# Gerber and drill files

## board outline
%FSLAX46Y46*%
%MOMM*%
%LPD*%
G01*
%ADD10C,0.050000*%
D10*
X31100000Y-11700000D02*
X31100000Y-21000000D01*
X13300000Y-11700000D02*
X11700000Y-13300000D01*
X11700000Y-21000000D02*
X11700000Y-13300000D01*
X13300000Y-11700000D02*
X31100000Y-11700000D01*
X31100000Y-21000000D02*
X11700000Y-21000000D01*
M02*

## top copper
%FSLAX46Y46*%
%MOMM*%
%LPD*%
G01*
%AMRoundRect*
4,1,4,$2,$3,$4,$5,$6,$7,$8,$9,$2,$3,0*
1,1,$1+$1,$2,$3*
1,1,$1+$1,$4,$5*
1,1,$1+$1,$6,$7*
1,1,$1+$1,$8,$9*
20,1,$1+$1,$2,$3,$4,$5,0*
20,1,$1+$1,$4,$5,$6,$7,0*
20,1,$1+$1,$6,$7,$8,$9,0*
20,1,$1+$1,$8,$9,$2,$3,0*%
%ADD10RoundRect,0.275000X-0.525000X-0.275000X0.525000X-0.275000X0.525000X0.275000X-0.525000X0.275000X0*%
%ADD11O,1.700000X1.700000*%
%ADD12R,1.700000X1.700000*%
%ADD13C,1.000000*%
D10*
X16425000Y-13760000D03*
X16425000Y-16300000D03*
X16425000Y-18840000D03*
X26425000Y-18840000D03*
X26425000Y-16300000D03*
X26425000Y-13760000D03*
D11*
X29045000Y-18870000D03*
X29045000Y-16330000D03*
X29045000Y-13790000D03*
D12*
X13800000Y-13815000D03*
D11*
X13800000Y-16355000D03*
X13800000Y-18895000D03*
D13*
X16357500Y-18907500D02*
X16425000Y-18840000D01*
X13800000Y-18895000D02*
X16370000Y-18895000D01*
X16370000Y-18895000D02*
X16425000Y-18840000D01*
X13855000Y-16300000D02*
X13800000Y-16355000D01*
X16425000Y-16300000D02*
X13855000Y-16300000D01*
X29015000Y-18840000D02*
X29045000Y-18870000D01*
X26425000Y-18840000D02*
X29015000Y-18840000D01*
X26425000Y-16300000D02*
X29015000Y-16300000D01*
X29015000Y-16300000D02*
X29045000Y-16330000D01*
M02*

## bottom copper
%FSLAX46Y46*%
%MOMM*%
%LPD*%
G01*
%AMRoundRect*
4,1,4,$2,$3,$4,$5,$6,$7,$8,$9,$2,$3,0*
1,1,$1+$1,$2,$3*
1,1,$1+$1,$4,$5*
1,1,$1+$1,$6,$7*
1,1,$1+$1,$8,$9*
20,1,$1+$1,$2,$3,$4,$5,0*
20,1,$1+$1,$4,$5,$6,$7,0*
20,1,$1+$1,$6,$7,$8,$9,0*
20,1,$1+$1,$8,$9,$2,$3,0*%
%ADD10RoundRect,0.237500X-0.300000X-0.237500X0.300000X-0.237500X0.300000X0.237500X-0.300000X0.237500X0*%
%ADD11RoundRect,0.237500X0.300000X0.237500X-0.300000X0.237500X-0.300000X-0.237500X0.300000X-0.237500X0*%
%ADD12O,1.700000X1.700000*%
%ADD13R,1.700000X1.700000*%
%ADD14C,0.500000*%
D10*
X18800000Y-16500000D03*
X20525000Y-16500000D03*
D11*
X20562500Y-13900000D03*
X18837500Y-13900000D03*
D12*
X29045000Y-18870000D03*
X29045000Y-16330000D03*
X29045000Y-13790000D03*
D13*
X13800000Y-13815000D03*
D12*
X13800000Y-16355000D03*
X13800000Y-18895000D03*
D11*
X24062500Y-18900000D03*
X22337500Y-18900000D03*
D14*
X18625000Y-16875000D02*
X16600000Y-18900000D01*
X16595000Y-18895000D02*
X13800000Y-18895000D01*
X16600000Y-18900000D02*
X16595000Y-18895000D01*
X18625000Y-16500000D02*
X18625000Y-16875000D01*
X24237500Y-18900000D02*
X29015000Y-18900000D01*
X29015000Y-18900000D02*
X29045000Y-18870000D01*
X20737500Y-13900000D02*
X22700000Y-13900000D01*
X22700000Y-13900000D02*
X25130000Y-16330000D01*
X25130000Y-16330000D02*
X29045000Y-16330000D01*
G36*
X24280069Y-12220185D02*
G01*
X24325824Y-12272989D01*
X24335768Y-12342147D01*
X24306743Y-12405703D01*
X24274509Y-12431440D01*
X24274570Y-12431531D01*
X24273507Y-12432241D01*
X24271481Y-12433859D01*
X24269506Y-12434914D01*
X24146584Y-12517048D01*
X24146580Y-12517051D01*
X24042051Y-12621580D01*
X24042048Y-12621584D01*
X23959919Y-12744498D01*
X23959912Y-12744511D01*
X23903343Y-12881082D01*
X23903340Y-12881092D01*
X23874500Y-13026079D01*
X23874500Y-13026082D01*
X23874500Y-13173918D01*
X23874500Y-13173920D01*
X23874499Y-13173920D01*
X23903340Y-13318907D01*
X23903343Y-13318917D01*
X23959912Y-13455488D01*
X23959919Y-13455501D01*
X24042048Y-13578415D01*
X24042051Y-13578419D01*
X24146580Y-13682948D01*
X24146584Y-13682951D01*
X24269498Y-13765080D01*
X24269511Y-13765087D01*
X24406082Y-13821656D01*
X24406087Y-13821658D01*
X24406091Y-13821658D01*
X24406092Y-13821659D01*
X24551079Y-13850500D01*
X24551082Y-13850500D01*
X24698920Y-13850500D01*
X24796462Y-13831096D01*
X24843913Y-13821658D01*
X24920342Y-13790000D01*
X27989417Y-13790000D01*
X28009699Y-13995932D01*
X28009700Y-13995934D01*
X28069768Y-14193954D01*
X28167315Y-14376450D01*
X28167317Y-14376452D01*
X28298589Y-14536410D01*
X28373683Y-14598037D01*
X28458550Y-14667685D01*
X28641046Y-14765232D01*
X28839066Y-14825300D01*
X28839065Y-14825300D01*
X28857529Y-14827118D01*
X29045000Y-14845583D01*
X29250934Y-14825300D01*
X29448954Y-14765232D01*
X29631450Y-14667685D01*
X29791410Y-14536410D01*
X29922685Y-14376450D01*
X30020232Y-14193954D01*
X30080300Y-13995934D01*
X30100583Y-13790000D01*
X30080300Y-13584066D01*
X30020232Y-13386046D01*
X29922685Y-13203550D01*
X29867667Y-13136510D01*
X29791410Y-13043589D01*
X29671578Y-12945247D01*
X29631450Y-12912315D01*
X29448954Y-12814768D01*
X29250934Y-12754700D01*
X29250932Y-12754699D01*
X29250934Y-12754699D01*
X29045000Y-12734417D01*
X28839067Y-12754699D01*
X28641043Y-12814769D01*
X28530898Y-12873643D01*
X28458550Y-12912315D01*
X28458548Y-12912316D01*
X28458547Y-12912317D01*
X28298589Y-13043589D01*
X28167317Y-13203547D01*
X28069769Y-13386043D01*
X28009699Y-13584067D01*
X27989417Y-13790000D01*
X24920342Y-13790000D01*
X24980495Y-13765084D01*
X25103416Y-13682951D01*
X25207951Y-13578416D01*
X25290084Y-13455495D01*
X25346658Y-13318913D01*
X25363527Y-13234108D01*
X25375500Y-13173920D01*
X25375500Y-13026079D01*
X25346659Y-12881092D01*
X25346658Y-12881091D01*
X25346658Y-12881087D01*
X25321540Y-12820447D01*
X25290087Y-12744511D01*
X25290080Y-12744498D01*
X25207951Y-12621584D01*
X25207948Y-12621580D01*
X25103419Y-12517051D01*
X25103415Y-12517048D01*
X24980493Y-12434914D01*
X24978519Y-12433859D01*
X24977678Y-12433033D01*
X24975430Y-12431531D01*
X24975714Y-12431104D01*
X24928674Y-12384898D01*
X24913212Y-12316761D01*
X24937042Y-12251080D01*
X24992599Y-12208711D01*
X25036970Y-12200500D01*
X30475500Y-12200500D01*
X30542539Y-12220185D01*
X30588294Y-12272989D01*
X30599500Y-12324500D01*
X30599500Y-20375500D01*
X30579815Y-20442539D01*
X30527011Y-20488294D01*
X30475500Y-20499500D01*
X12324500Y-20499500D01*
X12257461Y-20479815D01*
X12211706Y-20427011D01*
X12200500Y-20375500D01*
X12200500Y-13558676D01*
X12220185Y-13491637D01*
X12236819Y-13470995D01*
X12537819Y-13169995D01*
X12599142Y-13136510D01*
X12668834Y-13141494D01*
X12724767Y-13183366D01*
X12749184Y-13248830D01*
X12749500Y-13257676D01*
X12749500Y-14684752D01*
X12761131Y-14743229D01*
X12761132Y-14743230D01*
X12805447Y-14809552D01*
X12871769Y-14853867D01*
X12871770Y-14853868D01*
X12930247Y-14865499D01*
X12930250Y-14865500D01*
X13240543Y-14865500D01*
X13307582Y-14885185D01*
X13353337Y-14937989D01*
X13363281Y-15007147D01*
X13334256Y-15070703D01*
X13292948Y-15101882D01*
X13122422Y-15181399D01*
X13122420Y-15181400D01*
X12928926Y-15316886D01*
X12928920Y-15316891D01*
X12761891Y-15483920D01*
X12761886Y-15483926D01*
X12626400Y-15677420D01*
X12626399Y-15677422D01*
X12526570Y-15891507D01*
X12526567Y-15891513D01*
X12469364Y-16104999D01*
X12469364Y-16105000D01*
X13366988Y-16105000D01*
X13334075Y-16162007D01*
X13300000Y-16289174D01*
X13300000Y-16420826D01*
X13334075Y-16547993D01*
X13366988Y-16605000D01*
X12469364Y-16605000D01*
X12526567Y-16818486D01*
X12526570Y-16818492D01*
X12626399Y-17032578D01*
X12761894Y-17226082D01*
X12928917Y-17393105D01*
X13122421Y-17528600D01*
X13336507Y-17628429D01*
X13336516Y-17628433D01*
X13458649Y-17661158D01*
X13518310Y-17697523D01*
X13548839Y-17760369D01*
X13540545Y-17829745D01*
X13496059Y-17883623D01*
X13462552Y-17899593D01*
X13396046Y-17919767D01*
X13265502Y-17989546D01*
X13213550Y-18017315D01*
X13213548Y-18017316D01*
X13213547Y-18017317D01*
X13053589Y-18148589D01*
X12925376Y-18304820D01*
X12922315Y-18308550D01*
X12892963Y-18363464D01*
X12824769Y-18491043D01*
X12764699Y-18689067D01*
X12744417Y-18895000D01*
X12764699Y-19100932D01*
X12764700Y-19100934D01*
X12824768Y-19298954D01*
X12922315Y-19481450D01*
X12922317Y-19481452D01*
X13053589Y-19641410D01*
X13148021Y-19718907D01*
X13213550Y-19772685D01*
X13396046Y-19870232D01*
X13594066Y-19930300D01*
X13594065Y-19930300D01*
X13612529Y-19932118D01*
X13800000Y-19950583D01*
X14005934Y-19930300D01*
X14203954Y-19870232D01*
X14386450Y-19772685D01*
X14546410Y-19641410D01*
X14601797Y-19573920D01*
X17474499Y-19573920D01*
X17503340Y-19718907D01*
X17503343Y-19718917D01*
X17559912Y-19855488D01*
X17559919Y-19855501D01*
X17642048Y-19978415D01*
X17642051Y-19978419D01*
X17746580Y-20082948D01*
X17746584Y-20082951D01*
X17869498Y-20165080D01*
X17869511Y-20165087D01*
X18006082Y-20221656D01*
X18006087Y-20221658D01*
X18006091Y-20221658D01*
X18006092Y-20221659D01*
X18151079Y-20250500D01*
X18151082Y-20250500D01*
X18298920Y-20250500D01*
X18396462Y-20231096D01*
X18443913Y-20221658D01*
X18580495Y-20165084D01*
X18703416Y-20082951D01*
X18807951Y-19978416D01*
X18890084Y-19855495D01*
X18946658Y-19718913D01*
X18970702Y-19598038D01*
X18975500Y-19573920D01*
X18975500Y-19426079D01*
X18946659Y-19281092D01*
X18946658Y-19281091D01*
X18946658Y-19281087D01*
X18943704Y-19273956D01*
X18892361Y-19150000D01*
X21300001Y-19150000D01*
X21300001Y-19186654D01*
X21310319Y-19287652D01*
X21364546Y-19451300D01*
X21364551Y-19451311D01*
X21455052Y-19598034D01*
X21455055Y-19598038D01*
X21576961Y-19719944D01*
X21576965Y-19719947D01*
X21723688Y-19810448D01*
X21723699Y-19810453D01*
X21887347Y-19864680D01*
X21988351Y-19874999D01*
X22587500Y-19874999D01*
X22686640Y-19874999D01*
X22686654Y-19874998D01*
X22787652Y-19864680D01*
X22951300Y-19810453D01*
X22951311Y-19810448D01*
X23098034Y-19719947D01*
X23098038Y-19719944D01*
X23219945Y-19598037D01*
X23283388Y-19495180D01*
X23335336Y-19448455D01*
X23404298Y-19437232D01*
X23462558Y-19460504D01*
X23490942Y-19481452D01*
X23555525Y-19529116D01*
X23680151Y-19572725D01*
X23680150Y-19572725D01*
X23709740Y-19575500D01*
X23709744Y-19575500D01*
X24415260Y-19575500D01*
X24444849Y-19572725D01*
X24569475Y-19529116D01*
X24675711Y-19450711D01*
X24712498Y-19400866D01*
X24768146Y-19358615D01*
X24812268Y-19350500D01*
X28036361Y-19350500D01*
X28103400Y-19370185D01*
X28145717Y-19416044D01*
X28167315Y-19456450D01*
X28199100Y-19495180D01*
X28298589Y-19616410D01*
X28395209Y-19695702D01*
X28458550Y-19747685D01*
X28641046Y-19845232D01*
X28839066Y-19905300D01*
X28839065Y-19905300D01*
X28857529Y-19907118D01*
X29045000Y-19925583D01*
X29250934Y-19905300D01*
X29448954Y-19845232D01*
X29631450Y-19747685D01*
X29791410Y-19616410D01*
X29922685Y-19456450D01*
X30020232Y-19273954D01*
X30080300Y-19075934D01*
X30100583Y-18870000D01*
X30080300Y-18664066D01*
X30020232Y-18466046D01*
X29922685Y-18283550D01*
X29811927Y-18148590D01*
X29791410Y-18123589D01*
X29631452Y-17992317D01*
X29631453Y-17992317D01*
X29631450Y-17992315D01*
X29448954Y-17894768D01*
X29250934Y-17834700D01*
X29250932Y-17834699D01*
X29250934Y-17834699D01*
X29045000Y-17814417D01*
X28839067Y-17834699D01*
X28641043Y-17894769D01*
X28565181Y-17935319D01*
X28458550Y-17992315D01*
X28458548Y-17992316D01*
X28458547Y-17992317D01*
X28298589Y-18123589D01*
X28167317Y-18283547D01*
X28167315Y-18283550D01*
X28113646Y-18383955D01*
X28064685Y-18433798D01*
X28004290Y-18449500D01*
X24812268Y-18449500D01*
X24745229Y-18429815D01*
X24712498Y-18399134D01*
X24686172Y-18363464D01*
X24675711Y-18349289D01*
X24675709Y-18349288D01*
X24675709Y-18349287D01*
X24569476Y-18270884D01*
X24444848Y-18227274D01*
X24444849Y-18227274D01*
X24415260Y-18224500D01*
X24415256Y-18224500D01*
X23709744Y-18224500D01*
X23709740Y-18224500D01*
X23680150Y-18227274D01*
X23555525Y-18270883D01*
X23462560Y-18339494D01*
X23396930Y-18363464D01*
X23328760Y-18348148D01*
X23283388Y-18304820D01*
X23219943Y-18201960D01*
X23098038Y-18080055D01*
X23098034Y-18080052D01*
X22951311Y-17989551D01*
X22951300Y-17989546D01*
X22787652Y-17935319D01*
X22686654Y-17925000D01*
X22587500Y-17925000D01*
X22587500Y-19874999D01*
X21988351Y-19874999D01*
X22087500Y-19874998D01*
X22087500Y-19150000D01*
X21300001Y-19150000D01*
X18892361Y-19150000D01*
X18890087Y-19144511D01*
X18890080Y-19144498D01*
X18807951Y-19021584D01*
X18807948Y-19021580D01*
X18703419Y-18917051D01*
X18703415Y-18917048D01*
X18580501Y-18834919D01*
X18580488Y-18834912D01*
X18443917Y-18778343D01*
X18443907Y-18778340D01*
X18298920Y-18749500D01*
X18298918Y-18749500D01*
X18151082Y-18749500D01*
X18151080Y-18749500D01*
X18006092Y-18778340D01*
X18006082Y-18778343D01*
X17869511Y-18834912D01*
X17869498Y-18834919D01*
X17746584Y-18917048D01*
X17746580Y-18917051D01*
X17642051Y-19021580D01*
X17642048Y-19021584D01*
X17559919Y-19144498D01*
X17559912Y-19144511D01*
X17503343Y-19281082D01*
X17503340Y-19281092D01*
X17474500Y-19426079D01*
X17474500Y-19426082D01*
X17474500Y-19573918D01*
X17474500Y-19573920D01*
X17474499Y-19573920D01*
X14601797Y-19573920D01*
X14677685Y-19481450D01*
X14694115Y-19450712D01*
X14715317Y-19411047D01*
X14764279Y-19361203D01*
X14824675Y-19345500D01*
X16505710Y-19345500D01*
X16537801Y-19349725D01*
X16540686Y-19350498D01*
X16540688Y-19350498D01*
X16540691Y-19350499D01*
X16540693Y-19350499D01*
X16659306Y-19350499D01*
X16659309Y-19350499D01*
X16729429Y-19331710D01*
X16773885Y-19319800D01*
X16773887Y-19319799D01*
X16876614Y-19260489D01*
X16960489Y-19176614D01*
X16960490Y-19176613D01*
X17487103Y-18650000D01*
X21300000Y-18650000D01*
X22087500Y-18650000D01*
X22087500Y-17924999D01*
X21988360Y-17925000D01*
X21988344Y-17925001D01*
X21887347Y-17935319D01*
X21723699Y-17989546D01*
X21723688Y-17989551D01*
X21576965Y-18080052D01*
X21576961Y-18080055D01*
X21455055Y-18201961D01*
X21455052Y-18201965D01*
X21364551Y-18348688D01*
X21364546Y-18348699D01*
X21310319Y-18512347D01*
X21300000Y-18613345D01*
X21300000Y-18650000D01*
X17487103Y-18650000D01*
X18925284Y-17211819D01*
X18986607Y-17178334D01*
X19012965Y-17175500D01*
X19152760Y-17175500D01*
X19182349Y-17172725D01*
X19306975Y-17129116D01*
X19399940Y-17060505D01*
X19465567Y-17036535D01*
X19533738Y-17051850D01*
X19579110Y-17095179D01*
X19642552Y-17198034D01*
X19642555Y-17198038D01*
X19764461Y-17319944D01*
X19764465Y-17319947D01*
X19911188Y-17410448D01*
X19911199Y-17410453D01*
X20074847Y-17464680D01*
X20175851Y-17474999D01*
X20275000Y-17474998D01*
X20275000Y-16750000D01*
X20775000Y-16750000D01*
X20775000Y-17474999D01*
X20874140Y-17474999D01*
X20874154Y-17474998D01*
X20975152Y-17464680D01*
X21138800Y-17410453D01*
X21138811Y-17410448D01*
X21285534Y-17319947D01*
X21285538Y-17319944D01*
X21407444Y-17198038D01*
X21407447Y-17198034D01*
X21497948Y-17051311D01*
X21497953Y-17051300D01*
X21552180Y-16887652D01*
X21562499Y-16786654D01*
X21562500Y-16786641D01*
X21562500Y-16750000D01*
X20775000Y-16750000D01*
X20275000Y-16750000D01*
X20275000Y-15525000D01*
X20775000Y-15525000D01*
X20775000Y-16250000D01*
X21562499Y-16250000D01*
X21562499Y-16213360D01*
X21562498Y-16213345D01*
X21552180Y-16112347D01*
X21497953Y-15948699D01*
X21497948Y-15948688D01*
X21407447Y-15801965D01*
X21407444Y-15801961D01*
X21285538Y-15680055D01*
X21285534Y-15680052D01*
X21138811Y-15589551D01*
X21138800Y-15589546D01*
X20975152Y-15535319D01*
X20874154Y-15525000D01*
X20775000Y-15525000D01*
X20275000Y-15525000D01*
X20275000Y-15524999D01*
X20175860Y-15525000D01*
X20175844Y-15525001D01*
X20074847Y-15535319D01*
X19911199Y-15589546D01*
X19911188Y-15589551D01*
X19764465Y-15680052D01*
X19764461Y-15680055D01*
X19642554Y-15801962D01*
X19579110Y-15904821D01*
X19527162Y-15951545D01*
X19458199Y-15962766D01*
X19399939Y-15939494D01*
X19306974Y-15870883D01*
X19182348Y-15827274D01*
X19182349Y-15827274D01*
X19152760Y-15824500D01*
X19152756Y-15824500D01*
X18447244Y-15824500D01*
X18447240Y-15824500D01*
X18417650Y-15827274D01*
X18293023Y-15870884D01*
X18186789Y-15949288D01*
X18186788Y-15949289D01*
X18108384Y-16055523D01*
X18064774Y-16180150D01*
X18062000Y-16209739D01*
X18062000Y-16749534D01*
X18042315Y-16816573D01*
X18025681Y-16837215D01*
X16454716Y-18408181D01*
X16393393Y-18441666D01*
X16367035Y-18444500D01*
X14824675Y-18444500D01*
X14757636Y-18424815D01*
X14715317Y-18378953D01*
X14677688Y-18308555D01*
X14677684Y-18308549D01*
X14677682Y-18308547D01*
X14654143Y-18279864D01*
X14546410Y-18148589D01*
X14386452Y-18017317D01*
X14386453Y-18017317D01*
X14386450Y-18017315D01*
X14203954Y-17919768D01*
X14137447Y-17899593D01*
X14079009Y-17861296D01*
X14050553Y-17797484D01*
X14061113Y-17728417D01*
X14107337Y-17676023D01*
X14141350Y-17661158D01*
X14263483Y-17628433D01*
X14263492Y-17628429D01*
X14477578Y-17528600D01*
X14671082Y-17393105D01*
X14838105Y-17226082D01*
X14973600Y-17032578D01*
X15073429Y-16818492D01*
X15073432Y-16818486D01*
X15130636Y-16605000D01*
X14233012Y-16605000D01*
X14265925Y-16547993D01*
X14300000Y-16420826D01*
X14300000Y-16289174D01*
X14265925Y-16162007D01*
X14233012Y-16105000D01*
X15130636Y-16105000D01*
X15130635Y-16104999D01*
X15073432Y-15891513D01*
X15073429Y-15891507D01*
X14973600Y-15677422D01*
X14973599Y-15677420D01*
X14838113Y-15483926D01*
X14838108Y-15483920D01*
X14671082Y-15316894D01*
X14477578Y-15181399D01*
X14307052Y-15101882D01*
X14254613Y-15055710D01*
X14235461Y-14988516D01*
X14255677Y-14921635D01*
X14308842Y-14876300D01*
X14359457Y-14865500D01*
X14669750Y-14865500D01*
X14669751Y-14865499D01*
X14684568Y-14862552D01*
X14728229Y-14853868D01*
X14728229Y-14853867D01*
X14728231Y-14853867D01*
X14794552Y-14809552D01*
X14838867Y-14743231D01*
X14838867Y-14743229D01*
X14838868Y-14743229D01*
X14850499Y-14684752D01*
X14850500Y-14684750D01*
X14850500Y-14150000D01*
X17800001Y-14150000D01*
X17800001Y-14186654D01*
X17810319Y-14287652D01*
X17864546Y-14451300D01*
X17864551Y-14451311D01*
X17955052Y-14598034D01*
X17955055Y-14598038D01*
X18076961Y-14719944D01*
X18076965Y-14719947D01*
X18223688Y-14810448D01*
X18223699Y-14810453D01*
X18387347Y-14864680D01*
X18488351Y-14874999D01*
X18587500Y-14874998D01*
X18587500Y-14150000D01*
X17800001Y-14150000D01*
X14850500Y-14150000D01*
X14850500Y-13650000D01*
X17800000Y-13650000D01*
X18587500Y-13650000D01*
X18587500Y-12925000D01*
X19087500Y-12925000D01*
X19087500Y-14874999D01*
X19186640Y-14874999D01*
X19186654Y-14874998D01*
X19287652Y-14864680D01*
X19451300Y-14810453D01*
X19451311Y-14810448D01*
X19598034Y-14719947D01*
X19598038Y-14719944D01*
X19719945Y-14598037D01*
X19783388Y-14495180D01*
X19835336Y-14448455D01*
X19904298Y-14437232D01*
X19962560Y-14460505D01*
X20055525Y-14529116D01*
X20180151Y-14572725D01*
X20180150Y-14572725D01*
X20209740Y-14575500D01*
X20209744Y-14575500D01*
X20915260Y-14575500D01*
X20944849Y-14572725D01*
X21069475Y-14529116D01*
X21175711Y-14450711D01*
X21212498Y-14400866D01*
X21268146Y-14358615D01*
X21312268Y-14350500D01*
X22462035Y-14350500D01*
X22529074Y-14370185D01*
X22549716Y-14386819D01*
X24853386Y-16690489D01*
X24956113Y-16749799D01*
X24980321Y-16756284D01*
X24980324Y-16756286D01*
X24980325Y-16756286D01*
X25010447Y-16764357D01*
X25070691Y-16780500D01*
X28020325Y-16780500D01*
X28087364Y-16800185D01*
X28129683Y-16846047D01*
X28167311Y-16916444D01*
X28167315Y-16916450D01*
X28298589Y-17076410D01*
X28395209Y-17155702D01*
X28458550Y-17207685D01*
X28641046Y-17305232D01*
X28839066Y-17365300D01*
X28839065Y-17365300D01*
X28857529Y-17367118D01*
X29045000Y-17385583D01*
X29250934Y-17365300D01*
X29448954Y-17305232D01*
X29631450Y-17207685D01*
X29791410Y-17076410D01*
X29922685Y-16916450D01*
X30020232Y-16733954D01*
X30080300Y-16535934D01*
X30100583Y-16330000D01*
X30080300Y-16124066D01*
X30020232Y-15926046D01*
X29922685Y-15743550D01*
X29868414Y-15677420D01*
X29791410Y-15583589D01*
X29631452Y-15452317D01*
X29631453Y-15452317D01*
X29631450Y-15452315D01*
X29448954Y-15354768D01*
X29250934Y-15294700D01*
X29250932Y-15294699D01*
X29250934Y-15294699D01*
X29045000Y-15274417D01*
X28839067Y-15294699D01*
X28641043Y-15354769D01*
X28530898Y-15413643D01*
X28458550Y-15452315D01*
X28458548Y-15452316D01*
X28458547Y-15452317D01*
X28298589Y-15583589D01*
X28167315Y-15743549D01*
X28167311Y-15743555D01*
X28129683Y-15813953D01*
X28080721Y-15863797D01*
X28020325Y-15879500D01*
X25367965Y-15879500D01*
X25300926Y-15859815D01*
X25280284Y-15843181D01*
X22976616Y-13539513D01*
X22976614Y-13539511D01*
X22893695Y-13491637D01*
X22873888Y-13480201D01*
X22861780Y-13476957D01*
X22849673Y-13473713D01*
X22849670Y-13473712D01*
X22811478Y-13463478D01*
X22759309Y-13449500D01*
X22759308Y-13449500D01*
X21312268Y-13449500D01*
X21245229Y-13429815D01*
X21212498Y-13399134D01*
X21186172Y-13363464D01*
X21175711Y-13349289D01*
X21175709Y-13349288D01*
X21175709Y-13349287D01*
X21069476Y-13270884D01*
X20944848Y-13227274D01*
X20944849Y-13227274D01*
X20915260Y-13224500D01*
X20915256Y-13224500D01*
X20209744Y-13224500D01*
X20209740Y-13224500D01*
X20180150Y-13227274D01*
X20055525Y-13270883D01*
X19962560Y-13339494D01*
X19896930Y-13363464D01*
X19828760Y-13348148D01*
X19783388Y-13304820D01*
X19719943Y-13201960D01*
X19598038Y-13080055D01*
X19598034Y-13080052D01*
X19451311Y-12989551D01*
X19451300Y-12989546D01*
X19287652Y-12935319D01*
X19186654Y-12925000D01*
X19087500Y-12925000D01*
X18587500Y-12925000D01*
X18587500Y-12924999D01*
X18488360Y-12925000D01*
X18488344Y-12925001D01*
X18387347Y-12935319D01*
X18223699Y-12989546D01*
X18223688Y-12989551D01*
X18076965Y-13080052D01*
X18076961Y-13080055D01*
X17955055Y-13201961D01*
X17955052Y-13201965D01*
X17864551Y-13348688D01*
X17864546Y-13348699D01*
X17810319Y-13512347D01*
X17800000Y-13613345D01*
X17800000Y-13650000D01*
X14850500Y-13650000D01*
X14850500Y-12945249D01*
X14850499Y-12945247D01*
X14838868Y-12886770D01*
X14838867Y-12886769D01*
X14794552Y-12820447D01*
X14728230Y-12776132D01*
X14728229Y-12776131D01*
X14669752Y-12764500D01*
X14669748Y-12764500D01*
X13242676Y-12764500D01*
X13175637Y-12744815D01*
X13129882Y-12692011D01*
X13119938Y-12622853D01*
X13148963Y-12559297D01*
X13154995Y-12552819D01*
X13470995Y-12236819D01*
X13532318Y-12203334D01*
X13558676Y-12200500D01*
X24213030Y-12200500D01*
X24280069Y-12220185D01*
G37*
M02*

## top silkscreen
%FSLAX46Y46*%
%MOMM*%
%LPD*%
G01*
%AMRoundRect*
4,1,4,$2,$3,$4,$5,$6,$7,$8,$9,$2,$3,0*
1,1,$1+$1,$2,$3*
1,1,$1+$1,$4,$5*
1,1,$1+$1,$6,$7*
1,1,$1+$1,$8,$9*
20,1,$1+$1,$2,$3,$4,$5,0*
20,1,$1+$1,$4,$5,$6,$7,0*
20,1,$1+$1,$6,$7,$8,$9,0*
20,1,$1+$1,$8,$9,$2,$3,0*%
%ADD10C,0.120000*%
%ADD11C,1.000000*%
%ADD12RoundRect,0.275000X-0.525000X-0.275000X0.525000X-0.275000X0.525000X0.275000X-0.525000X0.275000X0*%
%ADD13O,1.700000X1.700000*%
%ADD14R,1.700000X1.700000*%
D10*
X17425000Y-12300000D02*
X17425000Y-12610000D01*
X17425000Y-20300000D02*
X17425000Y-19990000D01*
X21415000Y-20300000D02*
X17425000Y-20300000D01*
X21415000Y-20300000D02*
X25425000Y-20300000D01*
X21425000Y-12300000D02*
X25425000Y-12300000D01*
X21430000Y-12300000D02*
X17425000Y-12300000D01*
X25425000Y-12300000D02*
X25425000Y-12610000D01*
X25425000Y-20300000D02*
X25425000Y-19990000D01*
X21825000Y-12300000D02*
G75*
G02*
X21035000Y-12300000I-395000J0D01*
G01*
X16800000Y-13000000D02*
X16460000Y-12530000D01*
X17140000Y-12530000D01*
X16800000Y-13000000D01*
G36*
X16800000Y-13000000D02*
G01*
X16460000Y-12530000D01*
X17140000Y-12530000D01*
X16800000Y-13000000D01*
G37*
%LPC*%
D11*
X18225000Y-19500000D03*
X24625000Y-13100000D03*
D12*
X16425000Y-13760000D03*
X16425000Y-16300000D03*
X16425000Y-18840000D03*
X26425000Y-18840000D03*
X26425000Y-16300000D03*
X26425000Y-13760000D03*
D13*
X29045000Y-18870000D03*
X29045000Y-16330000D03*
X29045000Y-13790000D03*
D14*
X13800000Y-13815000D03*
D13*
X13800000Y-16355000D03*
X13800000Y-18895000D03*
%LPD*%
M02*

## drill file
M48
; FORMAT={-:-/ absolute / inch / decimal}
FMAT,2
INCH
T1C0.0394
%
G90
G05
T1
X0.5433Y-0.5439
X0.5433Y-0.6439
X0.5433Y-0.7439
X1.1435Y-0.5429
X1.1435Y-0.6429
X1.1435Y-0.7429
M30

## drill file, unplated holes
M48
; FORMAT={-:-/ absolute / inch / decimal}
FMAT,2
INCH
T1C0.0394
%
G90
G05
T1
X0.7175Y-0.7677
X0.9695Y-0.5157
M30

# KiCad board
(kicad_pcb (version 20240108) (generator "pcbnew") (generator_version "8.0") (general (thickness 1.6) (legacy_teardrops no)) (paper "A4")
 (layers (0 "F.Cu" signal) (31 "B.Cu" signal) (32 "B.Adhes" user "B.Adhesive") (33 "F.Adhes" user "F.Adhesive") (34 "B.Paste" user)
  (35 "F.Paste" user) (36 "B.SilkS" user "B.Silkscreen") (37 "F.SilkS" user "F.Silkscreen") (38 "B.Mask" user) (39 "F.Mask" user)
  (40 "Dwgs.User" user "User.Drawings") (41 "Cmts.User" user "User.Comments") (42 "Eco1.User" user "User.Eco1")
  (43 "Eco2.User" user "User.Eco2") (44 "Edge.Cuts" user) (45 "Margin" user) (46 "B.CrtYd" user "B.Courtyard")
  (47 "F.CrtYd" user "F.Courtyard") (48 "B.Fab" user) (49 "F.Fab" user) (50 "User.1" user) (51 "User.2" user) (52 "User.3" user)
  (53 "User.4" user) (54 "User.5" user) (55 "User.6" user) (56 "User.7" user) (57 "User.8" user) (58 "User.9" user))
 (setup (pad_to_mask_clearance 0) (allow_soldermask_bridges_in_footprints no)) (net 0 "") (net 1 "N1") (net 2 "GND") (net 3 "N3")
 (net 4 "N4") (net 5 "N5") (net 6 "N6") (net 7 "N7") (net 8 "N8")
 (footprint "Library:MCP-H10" (layer "F.Cu") (at 21.425 16.3)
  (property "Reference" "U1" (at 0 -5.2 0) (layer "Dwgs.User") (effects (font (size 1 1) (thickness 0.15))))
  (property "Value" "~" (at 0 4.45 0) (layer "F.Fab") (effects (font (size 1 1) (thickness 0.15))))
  (fp_line (start -4 -4) (end -4 -3.69) (stroke (width 0.12) (type solid)) (layer "F.SilkS"))
  (fp_line (start -4 4) (end -4 3.69) (stroke (width 0.12) (type solid)) (layer "F.SilkS"))
  (fp_line (start -0.01 4) (end -4 4) (stroke (width 0.12) (type solid)) (layer "F.SilkS"))
  (fp_line (start -0.01 4) (end 4 4) (stroke (width 0.12) (type solid)) (layer "F.SilkS"))
  (fp_line (start 0 -4) (end 4 -4) (stroke (width 0.12) (type solid)) (layer "F.SilkS"))
  (fp_line (start 0.005 -4) (end -4 -4) (stroke (width 0.12) (type solid)) (layer "F.SilkS"))
  (fp_line (start 4 -4) (end 4 -3.69) (stroke (width 0.12) (type solid)) (layer "F.SilkS"))
  (fp_line (start 4 4) (end 4 3.69) (stroke (width 0.12) (type solid)) (layer "F.SilkS"))
  (fp_arc (start 0.4 -4) (mid 0.005 -3.605) (end -0.39 -4) (stroke (width 0.12) (type default)) (layer "F.SilkS"))
  (fp_poly
   (pts (xy -4.625 -3.3) (xy -4.965 -3.77) (xy -4.285 -3.77) (xy -4.625 -3.3)) (stroke (width 0.12) (type solid)) (fill solid)
   (layer "F.SilkS"))
  (pad "" np_thru_hole circle (at -3.2 3.2) (size 1 1) (drill 1) (layers "F&B.Cu" "*.Mask"))
  (pad "" np_thru_hole circle (at 3.2 -3.2) (size 1 1) (drill 1) (layers "F&B.Cu" "*.Mask"))
  (pad "1" smd roundrect (at -5 -2.54) (size 1.6 1.1) (layers "F.Cu" "F.Paste" "F.Mask") (roundrect_rratio 0.25) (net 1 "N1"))
  (pad "2" smd roundrect (at -5 0) (size 1.6 1.1) (layers "F.Cu" "F.Paste" "F.Mask") (roundrect_rratio 0.25) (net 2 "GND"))
  (pad "3" smd roundrect (at -5 2.54) (size 1.6 1.1) (layers "F.Cu" "F.Paste" "F.Mask") (roundrect_rratio 0.25) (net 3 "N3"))
  (pad "4" smd roundrect (at 5 2.54) (size 1.6 1.1) (layers "F.Cu" "F.Paste" "F.Mask") (roundrect_rratio 0.25) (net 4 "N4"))
  (pad "5" smd roundrect (at 5 0) (size 1.6 1.1) (layers "F.Cu" "F.Paste" "F.Mask") (roundrect_rratio 0.25) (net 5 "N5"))
  (pad "6" smd roundrect (at 5 -2.54) (size 1.6 1.1) (layers "F.Cu" "F.Paste" "F.Mask") (roundrect_rratio 0.25) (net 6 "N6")))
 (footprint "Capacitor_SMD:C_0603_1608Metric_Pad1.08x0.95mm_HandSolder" (layer "B.Cu") (at 19.6625 16.5)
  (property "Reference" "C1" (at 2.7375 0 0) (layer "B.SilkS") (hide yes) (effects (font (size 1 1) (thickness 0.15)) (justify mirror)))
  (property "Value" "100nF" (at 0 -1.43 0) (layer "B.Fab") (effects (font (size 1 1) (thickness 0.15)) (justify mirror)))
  (pad "1" smd roundrect (at -0.8625 0) (size 1.075 0.95) (layers "B.Cu" "B.Paste" "B.Mask") (roundrect_rratio 0.25) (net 3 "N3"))
  (pad "2" smd roundrect (at 0.8625 0) (size 1.075 0.95) (layers "B.Cu" "B.Paste" "B.Mask") (roundrect_rratio 0.25) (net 2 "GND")))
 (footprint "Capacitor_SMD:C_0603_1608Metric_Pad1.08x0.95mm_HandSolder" (layer "B.Cu") (at 19.7 13.9 180)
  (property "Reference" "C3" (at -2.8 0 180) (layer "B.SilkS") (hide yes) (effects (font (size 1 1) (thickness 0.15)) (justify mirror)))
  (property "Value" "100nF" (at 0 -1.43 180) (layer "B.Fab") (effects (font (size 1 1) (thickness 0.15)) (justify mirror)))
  (pad "1" smd roundrect (at -0.8625 0 180) (size 1.075 0.95) (layers "B.Cu" "B.Paste" "B.Mask") (roundrect_rratio 0.25) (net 5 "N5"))
  (pad "2" smd roundrect (at 0.8625 0 180) (size 1.075 0.95) (layers "B.Cu" "B.Paste" "B.Mask") (roundrect_rratio 0.25) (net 2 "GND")))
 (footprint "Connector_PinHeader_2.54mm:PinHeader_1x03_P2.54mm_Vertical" (layer "B.Cu") (at 29.045 18.87)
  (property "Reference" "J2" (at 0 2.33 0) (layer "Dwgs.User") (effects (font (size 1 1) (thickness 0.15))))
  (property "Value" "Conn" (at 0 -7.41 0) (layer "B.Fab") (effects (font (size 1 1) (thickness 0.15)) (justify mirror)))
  (pad "1" thru_hole oval (at 0 0) (size 1.7 1.7) (drill 1) (layers "*.Cu" "*.Mask") (remove_unused_layers no) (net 4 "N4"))
  (pad "2" thru_hole oval (at 0 -2.54) (size 1.7 1.7) (drill 1) (layers "*.Cu" "*.Mask") (remove_unused_layers no) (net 5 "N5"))
  (pad "3" thru_hole oval (at 0 -5.08) (size 1.7 1.7) (drill 1) (layers "*.Cu" "*.Mask") (remove_unused_layers no) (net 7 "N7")))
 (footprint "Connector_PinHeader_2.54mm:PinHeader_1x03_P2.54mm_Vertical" (layer "B.Cu") (at 13.8 13.815 180)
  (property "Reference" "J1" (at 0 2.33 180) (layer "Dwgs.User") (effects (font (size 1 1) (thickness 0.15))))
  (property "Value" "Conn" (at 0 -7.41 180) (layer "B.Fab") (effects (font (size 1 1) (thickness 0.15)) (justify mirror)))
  (pad "1" thru_hole rect (at 0 0 180) (size 1.7 1.7) (drill 1) (layers "*.Cu" "*.Mask") (remove_unused_layers no) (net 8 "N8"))
  (pad "2" thru_hole oval (at 0 -2.54 180) (size 1.7 1.7) (drill 1) (layers "*.Cu" "*.Mask") (remove_unused_layers no) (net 2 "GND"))
  (pad "3" thru_hole oval (at 0 -5.08 180) (size 1.7 1.7) (drill 1) (layers "*.Cu" "*.Mask") (remove_unused_layers no) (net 3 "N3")))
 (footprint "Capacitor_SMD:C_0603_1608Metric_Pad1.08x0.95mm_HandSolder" (layer "B.Cu") (at 23.2 18.9 180)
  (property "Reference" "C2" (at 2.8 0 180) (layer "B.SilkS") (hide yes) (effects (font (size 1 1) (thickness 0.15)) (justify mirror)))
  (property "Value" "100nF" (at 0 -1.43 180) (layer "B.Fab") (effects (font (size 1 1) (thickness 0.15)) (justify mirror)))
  (pad "1" smd roundrect (at -0.8625 0 180) (size 1.075 0.95) (layers "B.Cu" "B.Paste" "B.Mask") (roundrect_rratio 0.25) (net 4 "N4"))
  (pad "2" smd roundrect (at 0.8625 0 180) (size 1.075 0.95) (layers "B.Cu" "B.Paste" "B.Mask") (roundrect_rratio 0.25) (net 2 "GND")))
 (gr_line (start 31.1 11.7) (end 31.1 21) (stroke (width 0.05) (type default)) (layer "Edge.Cuts"))
 (gr_line (start 13.3 11.7) (end 11.7 13.3) (stroke (width 0.05) (type default)) (layer "Edge.Cuts"))
 (gr_line (start 11.7 21) (end 11.7 13.3) (stroke (width 0.05) (type default)) (layer "Edge.Cuts"))
 (gr_line (start 13.3 11.7) (end 31.1 11.7) (stroke (width 0.05) (type default)) (layer "Edge.Cuts"))
 (gr_line (start 31.1 21) (end 11.7 21) (stroke (width 0.05) (type default)) (layer "Edge.Cuts"))
 (segment (start 16.3575 18.9075) (end 16.425 18.84) (width 1) (layer "F.Cu") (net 3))
 (segment (start 13.8 18.895) (end 16.37 18.895) (width 1) (layer "F.Cu") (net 3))
 (segment (start 16.37 18.895) (end 16.425 18.84) (width 1) (layer "F.Cu") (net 3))
 (segment (start 18.625 16.875) (end 16.6 18.9) (width 0.5) (layer "B.Cu") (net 3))
 (segment (start 16.595 18.895) (end 13.8 18.895) (width 0.5) (layer "B.Cu") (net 3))
 (segment (start 16.6 18.9) (end 16.595 18.895) (width 0.5) (layer "B.Cu") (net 3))
 (segment (start 18.625 16.5) (end 18.625 16.875) (width 0.5) (layer "B.Cu") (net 3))
 (segment (start 13.855 16.3) (end 13.8 16.355) (width 1) (layer "F.Cu") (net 2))
 (segment (start 16.425 16.3) (end 13.855 16.3) (width 1) (layer "F.Cu") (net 2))
 (segment (start 29.015 18.84) (end 29.045 18.87) (width 1) (layer "F.Cu") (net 4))
 (segment (start 26.425 18.84) (end 29.015 18.84) (width 1) (layer "F.Cu") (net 4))
 (segment (start 24.2375 18.9) (end 29.015 18.9) (width 0.5) (layer "B.Cu") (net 4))
 (segment (start 29.015 18.9) (end 29.045 18.87) (width 0.5) (layer "B.Cu") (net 4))
 (segment (start 26.425 16.3) (end 29.015 16.3) (width 1) (layer "F.Cu") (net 5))
 (segment (start 29.015 16.3) (end 29.045 16.33) (width 1) (layer "F.Cu") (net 5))
 (segment (start 20.7375 13.9) (end 22.7 13.9) (width 0.5) (layer "B.Cu") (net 5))
 (segment (start 22.7 13.9) (end 25.13 16.33) (width 0.5) (layer "B.Cu") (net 5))
 (segment (start 25.13 16.33) (end 29.045 16.33) (width 0.5) (layer "B.Cu") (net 5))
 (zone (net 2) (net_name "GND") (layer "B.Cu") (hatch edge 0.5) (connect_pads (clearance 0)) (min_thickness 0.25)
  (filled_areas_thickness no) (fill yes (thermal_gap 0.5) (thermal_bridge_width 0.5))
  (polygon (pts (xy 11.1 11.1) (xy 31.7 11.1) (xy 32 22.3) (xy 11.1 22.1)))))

